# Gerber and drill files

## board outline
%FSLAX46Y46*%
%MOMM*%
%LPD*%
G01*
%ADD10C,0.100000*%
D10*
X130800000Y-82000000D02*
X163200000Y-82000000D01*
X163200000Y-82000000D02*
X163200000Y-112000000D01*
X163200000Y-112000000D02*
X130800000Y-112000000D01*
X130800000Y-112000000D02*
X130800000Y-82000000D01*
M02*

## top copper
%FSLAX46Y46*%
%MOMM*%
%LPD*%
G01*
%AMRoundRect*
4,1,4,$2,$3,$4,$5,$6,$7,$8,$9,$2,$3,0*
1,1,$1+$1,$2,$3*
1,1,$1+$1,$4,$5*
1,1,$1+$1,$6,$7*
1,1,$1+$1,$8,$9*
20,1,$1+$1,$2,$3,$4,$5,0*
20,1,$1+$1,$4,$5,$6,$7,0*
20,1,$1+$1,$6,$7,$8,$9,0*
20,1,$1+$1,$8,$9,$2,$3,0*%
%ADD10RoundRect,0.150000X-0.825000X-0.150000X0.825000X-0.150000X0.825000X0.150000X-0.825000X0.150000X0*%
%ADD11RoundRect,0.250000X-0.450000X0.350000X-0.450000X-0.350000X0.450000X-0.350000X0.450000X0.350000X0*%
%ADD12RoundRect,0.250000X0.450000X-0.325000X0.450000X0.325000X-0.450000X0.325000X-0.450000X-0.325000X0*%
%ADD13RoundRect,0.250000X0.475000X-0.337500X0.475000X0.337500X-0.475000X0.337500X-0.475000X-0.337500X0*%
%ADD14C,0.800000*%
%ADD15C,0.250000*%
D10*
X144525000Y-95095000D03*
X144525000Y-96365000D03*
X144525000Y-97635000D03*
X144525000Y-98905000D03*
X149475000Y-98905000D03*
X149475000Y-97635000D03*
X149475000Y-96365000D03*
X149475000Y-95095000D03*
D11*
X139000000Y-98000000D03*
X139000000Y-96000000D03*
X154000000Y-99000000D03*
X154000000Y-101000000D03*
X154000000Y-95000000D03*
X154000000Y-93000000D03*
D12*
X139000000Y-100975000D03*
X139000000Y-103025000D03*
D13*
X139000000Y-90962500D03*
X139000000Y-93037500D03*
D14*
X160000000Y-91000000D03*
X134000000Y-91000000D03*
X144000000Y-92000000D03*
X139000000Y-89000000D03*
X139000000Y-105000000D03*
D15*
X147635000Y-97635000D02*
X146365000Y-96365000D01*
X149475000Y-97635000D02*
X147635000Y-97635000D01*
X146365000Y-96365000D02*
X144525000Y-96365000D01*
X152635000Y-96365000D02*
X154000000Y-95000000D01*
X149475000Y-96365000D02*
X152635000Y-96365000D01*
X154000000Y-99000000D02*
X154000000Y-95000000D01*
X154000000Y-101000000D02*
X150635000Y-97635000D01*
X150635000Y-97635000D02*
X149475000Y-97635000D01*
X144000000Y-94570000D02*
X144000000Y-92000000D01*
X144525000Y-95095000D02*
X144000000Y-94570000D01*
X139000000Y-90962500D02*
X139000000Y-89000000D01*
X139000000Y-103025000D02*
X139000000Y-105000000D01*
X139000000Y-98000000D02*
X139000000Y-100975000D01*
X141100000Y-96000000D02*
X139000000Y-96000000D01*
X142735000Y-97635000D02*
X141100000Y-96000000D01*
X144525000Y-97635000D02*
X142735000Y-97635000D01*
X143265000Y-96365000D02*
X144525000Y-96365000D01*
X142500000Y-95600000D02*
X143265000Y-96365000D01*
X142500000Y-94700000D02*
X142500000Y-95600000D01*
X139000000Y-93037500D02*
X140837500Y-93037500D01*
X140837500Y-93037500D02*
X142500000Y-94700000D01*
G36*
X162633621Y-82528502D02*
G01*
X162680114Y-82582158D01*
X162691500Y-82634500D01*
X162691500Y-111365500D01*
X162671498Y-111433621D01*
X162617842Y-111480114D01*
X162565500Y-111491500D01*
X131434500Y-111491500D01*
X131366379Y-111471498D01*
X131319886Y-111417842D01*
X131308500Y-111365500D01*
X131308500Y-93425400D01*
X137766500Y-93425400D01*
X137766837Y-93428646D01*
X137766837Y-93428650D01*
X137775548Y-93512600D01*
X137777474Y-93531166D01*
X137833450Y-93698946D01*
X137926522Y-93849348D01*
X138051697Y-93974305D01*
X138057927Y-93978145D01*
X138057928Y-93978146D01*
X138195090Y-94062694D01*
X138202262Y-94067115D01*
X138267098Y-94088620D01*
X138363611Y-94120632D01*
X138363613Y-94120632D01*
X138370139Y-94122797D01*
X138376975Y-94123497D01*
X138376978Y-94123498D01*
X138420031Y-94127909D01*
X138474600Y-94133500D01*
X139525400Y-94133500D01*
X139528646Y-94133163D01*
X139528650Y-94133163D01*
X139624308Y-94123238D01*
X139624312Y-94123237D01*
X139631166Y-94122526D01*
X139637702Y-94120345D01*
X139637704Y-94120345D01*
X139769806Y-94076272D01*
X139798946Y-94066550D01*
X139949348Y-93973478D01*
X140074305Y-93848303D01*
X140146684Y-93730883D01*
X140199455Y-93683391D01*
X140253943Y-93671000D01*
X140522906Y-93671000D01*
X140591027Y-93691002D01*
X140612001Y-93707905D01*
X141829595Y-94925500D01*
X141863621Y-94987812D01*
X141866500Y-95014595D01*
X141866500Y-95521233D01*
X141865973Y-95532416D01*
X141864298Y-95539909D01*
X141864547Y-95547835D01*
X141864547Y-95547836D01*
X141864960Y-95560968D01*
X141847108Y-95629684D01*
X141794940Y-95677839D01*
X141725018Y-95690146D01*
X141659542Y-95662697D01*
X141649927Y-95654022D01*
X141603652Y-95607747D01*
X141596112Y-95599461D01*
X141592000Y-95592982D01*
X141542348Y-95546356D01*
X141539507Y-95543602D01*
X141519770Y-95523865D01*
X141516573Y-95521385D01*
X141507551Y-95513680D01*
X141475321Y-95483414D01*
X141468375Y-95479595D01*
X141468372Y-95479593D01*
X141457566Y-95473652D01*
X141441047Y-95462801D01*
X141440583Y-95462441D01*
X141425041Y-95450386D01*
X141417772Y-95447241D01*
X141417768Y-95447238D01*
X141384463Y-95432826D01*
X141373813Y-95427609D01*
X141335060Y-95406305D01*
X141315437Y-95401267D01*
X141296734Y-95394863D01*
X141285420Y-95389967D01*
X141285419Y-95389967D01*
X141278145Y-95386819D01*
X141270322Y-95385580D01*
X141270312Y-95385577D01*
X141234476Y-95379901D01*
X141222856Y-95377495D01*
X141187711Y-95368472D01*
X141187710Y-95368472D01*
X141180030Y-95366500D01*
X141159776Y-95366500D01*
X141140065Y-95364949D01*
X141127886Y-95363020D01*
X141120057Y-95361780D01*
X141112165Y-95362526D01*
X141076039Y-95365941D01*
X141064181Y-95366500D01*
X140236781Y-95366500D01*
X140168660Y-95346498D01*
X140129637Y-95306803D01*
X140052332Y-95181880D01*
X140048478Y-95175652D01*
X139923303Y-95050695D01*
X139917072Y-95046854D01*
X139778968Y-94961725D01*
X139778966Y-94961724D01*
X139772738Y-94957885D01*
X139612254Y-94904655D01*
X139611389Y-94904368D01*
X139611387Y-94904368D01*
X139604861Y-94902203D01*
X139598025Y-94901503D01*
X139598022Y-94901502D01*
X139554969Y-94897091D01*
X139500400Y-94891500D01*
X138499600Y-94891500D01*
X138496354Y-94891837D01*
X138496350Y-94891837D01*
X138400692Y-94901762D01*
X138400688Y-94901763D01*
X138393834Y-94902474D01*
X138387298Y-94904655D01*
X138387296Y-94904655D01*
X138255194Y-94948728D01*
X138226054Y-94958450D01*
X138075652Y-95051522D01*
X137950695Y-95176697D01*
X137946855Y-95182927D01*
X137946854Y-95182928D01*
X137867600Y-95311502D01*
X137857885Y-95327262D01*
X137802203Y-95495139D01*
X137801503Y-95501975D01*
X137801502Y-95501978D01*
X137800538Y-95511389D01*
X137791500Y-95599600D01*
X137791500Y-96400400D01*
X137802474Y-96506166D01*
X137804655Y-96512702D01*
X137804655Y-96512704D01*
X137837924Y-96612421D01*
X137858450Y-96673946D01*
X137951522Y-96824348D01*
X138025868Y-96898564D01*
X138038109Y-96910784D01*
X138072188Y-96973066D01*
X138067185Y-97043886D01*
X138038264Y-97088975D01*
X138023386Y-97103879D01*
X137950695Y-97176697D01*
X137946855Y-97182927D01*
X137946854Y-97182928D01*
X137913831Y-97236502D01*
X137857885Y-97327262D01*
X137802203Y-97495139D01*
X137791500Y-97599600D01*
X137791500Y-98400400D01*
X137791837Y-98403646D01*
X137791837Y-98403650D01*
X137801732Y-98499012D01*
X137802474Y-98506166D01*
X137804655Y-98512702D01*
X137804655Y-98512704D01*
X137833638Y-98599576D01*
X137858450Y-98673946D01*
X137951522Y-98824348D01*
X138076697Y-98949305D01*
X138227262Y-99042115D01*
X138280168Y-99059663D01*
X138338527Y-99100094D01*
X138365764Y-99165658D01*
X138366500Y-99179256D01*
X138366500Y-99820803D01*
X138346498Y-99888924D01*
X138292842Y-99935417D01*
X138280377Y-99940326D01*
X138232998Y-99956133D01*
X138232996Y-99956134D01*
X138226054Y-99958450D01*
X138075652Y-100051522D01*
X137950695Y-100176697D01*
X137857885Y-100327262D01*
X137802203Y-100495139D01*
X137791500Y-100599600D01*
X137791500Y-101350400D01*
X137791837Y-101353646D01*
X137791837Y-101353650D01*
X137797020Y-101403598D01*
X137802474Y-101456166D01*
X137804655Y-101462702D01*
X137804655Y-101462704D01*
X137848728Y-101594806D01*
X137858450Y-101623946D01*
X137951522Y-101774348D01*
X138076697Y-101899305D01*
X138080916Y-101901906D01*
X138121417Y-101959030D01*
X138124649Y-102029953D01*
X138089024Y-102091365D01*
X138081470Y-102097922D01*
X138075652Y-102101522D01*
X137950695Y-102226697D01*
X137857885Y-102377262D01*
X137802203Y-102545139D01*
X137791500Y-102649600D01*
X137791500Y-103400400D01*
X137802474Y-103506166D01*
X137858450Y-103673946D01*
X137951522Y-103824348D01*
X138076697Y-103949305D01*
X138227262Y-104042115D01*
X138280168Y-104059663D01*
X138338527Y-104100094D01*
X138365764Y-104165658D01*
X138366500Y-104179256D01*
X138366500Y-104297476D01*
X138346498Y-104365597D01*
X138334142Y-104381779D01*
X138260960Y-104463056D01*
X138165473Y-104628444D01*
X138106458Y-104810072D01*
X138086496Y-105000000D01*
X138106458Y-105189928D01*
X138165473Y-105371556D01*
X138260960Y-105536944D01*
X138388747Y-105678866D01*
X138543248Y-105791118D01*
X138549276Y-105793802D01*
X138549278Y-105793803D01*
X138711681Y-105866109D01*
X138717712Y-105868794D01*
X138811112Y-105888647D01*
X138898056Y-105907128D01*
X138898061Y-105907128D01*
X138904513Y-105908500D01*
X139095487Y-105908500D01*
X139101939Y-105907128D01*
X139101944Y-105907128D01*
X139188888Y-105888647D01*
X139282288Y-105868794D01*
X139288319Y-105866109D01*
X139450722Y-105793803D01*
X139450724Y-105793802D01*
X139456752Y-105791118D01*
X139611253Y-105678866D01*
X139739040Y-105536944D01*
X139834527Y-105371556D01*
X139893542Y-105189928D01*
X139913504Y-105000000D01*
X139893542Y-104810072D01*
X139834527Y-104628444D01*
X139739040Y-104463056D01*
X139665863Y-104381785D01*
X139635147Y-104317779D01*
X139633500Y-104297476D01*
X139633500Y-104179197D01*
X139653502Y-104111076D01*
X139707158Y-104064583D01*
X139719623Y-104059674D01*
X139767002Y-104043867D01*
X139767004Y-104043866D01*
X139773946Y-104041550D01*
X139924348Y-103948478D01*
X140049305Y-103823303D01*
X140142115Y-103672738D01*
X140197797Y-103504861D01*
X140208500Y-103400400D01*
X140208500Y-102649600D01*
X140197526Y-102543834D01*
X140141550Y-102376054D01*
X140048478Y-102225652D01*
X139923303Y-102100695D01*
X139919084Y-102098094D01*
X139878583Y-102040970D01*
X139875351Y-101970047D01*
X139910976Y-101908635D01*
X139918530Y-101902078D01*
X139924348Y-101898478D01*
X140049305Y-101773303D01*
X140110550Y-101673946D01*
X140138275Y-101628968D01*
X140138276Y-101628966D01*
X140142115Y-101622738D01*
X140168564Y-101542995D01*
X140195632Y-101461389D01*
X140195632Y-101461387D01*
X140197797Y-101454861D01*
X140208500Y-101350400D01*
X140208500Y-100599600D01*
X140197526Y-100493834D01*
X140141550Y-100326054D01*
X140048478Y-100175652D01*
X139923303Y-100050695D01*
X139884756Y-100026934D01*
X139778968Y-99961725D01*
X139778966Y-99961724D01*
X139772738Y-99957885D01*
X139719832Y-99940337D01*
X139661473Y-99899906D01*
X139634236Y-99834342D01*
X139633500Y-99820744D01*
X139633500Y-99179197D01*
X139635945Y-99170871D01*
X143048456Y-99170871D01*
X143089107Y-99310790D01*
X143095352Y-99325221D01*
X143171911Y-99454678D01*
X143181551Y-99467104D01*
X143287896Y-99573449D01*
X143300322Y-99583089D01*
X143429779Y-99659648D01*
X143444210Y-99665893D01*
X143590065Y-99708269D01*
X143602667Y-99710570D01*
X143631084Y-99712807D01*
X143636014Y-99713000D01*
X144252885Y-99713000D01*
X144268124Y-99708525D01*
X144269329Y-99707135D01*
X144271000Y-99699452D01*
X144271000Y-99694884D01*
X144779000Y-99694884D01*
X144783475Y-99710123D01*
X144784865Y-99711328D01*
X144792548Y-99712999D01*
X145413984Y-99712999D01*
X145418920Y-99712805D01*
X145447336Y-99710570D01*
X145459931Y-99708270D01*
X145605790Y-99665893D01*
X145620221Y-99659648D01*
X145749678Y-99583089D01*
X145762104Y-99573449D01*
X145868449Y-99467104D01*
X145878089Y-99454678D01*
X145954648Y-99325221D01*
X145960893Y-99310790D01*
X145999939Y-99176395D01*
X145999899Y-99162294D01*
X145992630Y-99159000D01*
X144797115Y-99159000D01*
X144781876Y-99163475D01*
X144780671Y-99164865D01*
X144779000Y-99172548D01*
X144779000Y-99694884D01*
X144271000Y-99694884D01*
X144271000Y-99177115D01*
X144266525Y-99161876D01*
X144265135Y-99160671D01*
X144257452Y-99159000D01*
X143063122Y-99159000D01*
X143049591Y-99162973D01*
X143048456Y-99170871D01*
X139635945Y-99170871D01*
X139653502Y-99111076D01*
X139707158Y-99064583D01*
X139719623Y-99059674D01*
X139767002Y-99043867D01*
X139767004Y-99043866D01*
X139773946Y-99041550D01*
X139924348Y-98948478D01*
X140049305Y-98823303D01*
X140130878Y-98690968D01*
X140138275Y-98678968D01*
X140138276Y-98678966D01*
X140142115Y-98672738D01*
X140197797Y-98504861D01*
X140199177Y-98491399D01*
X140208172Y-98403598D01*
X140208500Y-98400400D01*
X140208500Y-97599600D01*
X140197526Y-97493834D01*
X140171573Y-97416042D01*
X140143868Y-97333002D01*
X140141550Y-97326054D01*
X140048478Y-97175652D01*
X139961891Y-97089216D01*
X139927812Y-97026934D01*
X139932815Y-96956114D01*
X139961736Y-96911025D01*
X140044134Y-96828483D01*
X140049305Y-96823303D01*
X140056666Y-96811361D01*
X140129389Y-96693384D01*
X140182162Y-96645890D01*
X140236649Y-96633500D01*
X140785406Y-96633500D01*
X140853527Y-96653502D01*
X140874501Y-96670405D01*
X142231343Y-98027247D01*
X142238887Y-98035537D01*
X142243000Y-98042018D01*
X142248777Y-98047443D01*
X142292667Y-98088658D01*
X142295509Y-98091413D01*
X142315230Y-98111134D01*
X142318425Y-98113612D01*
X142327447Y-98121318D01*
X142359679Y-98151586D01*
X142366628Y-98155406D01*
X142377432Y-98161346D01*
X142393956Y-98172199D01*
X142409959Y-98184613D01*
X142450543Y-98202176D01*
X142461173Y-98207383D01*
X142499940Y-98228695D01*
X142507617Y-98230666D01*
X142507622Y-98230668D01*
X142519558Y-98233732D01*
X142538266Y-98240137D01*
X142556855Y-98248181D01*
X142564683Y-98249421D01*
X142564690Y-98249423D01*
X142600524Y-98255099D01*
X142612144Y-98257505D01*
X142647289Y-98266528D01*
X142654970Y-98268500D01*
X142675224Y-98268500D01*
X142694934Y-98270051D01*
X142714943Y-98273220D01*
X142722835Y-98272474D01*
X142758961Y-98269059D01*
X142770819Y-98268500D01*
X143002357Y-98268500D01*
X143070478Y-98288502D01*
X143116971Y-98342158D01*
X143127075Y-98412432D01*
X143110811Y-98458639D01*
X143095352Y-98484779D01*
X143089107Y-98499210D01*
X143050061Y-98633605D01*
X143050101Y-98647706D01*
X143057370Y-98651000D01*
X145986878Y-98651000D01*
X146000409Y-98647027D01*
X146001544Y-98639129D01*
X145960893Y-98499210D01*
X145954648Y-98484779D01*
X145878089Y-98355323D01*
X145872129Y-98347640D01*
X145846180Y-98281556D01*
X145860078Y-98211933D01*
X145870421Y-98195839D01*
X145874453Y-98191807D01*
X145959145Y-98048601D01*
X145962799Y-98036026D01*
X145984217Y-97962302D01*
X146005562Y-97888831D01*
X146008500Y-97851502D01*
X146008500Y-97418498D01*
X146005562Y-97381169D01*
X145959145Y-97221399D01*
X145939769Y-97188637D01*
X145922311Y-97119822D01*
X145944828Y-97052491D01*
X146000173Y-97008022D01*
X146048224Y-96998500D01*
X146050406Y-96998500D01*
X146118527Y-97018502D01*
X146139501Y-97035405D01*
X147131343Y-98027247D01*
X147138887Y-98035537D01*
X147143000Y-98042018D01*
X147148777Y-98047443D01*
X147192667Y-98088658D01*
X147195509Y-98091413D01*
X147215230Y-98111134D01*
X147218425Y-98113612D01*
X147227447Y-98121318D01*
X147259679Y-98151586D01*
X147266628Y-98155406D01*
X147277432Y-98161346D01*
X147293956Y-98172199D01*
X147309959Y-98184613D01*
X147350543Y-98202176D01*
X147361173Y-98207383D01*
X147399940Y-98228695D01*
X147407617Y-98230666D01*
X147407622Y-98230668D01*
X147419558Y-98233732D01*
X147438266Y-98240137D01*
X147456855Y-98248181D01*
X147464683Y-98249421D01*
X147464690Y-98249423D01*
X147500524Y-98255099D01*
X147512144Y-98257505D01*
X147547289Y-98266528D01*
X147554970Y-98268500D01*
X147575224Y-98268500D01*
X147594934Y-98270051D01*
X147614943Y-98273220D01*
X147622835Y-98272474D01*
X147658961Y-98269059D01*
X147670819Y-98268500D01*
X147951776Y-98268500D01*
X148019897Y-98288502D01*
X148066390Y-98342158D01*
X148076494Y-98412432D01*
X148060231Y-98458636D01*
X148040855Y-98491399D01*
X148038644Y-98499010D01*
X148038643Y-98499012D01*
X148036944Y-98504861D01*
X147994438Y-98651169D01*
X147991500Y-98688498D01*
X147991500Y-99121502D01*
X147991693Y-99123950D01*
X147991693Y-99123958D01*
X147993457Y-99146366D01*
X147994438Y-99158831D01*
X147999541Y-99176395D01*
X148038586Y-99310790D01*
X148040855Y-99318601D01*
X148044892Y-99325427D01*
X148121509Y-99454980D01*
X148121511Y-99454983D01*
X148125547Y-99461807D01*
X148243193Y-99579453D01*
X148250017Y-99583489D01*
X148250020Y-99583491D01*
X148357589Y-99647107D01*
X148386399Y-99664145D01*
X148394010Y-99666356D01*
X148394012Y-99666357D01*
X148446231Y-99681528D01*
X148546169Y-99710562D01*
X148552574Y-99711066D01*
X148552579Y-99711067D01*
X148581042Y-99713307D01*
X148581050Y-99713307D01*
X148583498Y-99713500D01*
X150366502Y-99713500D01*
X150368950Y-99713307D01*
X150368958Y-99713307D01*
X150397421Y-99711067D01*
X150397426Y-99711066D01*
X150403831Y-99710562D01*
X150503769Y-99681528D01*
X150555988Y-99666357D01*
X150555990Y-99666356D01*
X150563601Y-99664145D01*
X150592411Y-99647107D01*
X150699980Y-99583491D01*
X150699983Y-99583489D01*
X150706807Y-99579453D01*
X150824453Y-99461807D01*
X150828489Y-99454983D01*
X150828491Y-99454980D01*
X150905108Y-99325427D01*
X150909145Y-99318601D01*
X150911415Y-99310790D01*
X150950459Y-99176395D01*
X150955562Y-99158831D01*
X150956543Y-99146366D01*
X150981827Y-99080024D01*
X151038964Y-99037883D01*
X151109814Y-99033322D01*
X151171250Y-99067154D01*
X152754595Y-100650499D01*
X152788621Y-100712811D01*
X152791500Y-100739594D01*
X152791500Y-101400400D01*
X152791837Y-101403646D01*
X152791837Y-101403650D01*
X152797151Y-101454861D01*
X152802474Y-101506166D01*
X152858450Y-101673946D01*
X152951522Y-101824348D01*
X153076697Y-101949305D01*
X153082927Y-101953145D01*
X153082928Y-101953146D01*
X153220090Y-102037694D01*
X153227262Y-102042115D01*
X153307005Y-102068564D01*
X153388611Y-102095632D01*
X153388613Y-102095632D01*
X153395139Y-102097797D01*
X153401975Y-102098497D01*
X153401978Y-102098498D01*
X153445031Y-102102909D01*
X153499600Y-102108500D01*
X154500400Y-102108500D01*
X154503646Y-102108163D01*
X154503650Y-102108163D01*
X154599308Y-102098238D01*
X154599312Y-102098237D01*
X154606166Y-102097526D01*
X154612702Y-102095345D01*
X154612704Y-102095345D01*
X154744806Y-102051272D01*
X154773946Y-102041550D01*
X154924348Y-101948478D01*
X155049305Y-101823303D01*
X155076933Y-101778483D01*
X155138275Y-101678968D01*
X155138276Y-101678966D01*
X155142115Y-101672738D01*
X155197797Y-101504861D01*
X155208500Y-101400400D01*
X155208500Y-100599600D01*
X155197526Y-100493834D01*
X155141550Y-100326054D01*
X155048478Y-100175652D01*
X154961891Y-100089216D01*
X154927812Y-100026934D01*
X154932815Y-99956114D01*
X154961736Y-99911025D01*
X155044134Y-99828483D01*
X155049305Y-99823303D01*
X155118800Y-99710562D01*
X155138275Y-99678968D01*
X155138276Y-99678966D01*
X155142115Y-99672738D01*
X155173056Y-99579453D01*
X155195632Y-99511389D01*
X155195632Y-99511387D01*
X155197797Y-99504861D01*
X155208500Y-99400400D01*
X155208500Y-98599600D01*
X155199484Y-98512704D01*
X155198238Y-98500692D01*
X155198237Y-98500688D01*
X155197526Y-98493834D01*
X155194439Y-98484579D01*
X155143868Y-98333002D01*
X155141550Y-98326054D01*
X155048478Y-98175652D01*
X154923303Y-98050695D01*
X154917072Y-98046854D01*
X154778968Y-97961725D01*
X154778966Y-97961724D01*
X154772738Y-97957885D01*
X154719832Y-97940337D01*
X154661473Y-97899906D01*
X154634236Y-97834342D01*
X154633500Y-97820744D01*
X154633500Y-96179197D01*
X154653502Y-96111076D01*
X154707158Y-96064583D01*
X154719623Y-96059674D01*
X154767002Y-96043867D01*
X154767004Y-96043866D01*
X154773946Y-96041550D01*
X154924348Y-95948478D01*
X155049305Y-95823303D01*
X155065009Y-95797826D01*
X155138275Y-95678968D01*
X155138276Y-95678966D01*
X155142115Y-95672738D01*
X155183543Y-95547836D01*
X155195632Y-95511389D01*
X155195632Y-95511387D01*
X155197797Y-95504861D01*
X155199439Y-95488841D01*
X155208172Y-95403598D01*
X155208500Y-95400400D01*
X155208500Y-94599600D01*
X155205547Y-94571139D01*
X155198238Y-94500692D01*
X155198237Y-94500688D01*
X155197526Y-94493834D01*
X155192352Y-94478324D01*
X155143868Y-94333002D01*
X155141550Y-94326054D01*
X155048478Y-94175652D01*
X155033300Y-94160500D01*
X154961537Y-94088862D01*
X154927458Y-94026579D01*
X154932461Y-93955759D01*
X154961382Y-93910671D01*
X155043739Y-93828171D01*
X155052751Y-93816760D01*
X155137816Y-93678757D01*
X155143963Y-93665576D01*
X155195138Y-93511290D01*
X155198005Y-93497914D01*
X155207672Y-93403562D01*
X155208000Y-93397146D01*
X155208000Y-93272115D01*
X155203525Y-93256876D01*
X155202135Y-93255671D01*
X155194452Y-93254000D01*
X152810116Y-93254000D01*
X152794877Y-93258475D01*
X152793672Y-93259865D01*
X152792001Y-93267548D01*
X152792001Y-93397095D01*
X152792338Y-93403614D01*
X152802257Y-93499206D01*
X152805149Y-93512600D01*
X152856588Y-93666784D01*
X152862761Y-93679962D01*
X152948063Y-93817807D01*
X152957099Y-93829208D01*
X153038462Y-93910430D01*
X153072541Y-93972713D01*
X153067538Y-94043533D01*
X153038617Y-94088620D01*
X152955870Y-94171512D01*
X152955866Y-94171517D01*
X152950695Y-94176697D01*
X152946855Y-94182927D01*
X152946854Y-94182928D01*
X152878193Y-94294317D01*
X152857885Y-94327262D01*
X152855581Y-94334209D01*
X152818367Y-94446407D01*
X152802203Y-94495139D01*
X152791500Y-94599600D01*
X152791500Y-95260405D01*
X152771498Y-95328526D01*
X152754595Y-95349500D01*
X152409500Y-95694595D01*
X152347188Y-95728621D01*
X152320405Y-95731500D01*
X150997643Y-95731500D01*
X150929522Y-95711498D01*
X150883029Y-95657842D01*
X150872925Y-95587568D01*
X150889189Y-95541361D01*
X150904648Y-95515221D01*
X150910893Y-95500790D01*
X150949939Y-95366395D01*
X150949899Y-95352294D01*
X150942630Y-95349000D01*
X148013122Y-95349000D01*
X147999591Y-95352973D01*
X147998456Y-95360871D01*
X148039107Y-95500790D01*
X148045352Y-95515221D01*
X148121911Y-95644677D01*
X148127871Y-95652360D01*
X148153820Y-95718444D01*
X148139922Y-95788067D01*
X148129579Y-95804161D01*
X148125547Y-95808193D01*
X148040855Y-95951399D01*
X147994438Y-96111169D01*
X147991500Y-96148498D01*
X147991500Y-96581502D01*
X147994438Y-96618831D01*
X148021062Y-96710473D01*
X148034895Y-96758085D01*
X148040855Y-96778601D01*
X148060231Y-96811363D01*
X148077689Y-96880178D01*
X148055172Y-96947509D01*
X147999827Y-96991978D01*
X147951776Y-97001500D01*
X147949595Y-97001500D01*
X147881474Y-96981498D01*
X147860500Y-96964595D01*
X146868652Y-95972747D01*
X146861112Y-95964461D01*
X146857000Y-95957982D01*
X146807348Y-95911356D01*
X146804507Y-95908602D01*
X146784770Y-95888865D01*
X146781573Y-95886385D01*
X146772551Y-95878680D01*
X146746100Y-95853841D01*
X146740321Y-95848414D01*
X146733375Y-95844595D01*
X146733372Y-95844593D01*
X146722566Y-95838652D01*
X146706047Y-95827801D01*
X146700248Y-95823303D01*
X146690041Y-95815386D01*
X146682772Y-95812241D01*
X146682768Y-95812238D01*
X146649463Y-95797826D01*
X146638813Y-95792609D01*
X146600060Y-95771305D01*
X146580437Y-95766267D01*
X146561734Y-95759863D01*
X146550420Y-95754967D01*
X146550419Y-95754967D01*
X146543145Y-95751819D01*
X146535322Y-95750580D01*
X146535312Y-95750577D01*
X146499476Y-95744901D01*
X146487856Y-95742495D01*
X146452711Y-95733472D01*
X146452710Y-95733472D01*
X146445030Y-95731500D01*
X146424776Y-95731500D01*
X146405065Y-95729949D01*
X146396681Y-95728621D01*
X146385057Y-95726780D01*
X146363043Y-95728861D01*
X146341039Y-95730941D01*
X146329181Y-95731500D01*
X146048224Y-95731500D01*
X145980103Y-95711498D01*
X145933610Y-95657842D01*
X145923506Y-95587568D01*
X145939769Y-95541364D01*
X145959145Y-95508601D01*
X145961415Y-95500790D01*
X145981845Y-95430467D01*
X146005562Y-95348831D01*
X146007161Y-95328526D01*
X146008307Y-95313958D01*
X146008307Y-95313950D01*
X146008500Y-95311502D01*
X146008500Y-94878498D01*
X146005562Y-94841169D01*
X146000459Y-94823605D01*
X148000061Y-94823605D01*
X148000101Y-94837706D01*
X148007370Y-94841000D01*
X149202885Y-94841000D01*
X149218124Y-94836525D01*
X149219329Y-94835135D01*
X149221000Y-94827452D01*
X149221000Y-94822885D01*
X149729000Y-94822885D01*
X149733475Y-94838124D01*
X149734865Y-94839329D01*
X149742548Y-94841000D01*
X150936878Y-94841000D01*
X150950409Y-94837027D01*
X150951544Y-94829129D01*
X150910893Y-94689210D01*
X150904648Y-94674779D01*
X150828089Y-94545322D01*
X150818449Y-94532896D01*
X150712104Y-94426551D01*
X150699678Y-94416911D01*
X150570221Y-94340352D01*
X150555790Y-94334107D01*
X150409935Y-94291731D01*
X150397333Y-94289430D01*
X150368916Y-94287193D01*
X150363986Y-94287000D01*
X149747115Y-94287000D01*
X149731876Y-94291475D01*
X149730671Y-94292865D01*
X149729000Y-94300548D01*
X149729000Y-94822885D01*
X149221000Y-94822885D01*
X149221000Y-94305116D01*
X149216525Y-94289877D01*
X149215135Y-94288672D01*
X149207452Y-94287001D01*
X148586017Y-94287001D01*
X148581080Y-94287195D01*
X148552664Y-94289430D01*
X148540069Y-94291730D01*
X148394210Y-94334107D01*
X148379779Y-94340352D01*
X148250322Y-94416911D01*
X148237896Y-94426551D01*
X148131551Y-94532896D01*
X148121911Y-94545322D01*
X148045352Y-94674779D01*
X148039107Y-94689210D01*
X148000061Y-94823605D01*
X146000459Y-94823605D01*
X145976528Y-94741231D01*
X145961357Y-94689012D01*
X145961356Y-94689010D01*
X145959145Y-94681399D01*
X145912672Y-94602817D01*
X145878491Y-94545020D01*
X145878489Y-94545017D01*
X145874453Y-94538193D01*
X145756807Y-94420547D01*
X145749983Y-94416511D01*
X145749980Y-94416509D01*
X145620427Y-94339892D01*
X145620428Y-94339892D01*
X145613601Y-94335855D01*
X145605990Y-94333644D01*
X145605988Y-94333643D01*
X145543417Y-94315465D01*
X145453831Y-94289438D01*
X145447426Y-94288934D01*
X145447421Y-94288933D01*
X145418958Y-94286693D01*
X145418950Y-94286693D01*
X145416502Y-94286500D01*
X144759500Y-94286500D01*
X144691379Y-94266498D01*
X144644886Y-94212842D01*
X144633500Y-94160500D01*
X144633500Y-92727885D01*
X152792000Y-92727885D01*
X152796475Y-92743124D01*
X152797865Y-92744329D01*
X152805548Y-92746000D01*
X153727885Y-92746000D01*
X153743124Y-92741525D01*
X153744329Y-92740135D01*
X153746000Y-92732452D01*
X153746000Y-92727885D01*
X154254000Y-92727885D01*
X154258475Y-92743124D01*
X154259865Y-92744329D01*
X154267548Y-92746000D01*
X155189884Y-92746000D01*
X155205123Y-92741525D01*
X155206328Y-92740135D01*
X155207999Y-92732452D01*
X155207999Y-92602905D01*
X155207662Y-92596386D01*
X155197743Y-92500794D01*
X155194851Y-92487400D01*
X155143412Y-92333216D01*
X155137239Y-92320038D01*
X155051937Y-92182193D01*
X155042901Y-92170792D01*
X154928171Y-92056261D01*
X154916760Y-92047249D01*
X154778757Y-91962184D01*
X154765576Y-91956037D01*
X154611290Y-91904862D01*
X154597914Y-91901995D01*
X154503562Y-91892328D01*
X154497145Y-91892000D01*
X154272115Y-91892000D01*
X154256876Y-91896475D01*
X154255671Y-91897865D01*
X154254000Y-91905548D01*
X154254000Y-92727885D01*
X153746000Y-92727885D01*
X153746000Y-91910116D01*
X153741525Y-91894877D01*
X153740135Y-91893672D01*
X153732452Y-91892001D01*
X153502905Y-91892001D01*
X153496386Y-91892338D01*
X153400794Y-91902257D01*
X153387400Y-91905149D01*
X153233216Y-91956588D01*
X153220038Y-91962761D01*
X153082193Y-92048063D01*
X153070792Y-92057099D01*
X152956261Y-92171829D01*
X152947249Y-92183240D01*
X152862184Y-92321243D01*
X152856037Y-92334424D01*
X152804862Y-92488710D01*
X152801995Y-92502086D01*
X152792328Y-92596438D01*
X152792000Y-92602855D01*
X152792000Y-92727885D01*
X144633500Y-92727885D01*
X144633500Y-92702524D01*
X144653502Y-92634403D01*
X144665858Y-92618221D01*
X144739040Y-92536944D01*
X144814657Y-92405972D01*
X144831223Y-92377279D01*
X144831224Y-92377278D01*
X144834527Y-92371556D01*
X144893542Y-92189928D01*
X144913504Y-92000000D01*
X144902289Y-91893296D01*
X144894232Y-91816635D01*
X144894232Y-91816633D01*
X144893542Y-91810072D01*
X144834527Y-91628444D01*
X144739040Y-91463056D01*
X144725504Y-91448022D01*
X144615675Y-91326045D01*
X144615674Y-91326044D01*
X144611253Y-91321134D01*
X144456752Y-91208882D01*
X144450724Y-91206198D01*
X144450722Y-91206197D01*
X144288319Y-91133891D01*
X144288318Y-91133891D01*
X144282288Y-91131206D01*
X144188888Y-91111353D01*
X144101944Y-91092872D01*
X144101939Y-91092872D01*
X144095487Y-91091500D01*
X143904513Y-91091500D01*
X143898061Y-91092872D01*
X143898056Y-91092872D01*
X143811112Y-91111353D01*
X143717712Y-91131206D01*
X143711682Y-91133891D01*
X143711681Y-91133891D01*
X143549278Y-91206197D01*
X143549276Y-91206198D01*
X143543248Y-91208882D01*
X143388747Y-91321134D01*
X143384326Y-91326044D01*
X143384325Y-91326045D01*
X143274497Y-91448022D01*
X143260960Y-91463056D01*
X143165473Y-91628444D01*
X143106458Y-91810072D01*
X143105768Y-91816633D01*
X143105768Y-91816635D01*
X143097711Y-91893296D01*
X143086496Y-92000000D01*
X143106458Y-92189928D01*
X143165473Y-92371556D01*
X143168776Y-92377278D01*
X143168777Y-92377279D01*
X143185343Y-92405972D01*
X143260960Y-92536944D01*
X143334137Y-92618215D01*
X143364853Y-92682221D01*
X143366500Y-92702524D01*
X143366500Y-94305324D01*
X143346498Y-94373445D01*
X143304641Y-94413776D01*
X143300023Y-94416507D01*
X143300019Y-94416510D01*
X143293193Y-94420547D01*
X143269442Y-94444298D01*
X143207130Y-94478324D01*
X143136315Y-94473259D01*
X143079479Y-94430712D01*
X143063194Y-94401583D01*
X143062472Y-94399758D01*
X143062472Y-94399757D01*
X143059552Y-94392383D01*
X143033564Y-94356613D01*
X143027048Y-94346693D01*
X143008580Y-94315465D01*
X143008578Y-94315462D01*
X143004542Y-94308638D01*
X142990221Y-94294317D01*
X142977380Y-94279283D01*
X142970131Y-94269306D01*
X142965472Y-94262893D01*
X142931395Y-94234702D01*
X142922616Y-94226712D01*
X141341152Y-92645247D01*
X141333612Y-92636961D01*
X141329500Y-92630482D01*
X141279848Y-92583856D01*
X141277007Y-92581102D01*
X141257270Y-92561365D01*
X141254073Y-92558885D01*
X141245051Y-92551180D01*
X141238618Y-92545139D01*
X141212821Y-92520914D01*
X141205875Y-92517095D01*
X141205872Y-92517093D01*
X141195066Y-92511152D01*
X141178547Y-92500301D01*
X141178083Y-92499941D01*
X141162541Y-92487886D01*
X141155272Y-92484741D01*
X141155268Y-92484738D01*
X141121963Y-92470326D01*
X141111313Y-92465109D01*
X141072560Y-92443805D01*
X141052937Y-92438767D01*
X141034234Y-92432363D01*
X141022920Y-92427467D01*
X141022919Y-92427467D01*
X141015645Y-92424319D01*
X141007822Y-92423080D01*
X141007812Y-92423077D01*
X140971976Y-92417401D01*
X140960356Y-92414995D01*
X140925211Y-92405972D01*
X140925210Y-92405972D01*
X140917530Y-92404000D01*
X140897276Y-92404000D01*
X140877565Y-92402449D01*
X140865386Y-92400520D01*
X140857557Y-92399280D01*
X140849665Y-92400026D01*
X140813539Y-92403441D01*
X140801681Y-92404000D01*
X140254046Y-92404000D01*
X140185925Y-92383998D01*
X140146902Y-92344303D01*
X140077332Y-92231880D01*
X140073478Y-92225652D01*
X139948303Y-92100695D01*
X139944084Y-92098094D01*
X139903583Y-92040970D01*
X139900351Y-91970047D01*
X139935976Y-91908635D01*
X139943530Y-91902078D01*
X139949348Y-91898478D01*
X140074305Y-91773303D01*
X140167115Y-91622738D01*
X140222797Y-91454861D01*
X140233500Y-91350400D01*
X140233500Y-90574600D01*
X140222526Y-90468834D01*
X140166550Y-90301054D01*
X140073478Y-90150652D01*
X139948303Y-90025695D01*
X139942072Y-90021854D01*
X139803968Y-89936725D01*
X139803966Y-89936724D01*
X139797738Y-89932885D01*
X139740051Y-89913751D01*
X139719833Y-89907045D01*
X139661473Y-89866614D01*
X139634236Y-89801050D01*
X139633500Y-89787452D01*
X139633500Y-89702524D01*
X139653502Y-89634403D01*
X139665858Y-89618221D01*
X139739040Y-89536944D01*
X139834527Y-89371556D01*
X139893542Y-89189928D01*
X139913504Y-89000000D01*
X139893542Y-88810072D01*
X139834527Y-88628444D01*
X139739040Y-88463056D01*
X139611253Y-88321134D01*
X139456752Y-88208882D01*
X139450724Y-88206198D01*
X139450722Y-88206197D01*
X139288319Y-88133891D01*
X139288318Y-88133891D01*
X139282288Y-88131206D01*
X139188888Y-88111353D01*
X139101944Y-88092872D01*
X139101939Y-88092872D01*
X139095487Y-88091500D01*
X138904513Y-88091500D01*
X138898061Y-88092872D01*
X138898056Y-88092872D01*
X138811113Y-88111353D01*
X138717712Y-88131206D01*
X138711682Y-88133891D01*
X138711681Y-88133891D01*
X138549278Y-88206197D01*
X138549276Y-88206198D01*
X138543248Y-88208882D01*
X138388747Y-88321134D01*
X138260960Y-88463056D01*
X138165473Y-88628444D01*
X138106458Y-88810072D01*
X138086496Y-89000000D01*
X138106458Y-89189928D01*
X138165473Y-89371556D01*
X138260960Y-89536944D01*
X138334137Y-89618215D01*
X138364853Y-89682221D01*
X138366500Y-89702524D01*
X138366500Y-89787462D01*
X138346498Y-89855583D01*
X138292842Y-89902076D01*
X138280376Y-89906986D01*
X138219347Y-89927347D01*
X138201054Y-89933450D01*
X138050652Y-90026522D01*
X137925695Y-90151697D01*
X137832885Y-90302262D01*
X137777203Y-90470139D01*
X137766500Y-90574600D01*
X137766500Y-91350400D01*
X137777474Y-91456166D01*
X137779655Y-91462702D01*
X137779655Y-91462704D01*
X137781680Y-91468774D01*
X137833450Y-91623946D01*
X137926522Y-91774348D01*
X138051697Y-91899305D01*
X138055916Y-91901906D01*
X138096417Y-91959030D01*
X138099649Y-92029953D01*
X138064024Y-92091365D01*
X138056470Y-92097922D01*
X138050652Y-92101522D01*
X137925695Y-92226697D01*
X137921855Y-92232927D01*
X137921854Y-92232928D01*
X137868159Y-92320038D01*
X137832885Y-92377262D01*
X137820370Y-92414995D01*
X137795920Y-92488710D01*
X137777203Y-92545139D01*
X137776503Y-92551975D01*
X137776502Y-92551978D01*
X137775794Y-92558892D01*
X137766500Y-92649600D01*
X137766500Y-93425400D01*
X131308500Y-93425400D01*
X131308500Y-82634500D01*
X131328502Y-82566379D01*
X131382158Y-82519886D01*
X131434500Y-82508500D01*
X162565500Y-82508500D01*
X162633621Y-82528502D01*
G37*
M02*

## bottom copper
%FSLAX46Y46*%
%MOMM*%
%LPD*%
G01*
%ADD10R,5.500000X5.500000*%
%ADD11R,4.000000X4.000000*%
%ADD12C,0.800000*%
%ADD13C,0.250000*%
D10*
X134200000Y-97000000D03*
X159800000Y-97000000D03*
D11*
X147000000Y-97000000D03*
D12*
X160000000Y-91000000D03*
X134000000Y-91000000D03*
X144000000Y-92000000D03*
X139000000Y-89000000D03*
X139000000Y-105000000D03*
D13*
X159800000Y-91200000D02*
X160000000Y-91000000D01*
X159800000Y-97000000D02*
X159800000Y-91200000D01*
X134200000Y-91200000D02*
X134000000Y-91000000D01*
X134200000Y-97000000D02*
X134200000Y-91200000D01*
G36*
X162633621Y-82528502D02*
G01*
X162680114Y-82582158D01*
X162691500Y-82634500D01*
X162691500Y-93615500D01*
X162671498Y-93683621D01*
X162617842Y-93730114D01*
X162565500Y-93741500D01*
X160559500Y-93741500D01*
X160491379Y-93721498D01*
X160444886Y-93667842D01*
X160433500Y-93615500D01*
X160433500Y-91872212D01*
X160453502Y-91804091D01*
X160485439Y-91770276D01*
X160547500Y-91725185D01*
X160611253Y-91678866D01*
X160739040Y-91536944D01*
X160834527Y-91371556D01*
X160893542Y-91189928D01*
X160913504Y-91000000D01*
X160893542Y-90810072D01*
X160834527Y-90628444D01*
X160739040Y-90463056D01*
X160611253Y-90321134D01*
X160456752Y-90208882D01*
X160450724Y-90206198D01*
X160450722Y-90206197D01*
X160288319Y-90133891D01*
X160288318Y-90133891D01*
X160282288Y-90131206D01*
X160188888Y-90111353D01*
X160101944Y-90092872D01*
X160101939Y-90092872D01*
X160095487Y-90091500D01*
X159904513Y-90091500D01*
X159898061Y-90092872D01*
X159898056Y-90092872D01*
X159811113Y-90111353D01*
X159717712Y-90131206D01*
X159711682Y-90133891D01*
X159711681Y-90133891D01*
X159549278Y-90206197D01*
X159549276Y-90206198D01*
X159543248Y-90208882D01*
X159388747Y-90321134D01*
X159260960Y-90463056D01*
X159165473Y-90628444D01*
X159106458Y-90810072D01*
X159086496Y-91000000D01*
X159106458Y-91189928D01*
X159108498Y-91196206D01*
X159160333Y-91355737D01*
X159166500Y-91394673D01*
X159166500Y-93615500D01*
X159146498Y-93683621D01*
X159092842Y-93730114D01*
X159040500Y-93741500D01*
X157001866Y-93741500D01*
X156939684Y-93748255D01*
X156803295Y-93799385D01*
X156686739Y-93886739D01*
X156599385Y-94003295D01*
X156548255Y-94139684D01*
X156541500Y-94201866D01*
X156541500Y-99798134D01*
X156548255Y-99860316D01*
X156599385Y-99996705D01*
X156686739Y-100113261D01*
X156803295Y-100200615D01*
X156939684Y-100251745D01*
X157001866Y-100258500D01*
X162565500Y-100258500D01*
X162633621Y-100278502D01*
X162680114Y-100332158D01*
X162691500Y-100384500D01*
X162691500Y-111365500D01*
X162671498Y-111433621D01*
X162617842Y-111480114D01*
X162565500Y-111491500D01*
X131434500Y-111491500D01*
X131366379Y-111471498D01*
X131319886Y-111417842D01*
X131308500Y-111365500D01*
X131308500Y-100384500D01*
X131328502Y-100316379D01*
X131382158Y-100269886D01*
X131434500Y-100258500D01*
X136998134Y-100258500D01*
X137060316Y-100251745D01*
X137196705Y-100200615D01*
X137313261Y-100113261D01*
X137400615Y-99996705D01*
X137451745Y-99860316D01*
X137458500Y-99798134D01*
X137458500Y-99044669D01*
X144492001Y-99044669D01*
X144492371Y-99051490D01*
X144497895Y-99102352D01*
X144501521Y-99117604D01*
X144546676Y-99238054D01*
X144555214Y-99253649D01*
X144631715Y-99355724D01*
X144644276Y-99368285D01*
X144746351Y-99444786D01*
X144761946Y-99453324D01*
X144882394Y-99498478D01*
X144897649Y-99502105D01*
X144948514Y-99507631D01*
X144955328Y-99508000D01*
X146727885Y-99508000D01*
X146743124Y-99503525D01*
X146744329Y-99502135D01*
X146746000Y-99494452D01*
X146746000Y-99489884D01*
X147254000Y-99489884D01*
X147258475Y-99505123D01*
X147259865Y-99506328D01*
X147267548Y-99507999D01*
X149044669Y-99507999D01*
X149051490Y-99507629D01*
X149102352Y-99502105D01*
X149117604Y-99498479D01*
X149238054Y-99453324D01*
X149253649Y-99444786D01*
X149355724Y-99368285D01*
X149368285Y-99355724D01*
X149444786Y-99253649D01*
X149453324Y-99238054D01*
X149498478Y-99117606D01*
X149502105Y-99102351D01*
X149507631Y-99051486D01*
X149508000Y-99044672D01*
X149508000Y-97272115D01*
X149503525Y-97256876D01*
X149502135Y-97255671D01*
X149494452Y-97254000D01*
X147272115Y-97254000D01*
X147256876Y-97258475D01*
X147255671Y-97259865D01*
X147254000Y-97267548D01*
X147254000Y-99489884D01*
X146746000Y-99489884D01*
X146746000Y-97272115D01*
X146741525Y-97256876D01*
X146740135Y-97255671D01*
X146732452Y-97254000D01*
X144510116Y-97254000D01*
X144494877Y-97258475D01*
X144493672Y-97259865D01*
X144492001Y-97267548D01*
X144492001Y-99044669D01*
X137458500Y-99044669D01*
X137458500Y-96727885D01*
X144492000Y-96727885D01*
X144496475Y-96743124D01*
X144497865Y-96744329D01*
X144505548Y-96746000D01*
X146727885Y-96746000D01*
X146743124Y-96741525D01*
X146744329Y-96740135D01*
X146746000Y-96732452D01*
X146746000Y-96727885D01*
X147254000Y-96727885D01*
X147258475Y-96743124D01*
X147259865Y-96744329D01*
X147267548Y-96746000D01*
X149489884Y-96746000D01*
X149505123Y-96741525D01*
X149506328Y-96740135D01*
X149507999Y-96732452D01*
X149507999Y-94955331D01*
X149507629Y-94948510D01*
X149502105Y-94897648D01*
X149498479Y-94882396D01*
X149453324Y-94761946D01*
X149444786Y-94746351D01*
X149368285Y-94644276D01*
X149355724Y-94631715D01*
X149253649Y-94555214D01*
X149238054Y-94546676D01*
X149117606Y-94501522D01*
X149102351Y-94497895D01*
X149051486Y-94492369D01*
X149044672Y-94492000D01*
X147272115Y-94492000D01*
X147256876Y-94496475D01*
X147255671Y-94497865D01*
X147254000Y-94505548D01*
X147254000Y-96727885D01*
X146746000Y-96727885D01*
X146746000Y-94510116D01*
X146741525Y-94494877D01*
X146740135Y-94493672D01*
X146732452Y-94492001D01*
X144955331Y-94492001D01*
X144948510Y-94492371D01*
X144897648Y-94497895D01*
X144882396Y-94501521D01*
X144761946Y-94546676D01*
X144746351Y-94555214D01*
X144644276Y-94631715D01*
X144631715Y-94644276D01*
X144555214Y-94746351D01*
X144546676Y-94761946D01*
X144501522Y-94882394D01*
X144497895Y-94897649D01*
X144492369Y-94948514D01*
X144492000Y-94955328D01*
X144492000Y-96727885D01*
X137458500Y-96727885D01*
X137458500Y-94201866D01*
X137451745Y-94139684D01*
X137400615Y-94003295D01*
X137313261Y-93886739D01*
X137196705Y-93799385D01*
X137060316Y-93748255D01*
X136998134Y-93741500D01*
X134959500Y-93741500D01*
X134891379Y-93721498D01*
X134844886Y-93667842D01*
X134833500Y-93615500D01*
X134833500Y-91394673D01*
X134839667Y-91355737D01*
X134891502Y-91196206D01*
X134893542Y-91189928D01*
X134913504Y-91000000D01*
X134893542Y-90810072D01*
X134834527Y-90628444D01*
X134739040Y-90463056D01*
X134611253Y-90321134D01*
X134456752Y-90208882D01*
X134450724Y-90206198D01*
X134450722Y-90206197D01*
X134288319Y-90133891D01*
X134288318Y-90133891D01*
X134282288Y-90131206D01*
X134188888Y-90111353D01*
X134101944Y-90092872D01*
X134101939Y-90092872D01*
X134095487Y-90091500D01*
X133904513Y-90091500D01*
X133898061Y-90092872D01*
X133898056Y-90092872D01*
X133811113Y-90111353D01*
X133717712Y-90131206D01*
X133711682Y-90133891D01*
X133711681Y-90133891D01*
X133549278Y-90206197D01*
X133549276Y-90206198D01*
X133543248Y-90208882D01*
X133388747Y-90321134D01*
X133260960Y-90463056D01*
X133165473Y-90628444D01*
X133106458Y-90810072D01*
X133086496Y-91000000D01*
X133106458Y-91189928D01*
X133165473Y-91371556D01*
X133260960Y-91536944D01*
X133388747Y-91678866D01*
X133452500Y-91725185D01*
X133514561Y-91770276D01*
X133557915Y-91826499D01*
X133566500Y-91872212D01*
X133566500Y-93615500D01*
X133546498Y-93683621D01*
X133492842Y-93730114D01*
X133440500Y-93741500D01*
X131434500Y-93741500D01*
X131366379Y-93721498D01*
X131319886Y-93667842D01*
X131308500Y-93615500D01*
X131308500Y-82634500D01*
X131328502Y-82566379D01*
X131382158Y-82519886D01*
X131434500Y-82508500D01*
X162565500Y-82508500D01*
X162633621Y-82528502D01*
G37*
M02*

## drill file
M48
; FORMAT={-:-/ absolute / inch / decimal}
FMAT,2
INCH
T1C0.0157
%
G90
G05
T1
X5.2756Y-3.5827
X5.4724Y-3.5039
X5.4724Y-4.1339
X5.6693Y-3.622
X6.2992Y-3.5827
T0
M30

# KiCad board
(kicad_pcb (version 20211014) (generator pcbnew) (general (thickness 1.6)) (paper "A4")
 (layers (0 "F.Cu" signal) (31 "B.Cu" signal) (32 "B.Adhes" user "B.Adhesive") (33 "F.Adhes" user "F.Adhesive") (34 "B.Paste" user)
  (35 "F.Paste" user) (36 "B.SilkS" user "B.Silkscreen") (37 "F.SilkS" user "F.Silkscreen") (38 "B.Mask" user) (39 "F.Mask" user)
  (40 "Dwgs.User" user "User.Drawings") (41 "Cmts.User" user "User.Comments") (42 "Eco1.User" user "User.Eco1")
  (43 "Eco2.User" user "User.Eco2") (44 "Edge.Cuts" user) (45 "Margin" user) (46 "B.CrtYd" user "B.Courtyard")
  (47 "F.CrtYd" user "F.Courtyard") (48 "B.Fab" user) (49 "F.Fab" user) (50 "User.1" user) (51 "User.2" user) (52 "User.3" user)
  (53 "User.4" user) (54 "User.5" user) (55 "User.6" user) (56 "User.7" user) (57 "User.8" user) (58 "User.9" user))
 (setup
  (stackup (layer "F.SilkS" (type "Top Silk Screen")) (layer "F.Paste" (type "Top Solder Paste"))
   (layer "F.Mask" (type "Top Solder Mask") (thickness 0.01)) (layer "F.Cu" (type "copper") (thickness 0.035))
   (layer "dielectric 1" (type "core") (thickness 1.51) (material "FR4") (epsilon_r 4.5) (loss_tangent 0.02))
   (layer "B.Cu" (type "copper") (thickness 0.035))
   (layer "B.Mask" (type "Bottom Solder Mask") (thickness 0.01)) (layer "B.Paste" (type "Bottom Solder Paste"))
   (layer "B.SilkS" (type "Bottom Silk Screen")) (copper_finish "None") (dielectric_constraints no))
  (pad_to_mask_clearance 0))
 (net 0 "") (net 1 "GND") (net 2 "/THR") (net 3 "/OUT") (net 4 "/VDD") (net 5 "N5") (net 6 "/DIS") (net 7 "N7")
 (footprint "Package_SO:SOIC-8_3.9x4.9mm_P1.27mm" (layer "F.Cu") (at 147 97)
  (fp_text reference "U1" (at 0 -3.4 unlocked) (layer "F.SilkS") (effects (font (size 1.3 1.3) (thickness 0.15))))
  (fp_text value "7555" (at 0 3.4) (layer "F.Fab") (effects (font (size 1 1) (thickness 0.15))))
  (pad "1" smd roundrect (at -2.475 -1.905) (size 1.95 0.6) (layers "F.Cu" "F.Paste" "F.Mask") (roundrect_rratio 0.25) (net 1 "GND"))
  (pad "2" smd roundrect (at -2.475 -0.635) (size 1.95 0.6) (layers "F.Cu" "F.Paste" "F.Mask") (roundrect_rratio 0.25) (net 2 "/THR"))
  (pad "3" smd roundrect (at -2.475 0.635) (size 1.95 0.6) (layers "F.Cu" "F.Paste" "F.Mask") (roundrect_rratio 0.25) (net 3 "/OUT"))
  (pad "4" smd roundrect (at -2.475 1.905) (size 1.95 0.6) (layers "F.Cu" "F.Paste" "F.Mask") (roundrect_rratio 0.25) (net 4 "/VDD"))
  (pad "5" smd roundrect (at 2.475 1.905) (size 1.95 0.6) (layers "F.Cu" "F.Paste" "F.Mask") (roundrect_rratio 0.25) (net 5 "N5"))
  (pad "6" smd roundrect (at 2.475 0.635) (size 1.95 0.6) (layers "F.Cu" "F.Paste" "F.Mask") (roundrect_rratio 0.25) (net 2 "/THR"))
  (pad "7" smd roundrect (at 2.475 -0.635) (size 1.95 0.6) (layers "F.Cu" "F.Paste" "F.Mask") (roundrect_rratio 0.25) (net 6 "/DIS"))
  (pad "8" smd roundrect (at 2.475 -1.905) (size 1.95 0.6) (layers "F.Cu" "F.Paste" "F.Mask") (roundrect_rratio 0.25) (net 4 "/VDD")))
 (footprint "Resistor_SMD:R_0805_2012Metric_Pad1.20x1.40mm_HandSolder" (layer "F.Cu") (at 154 94 -90)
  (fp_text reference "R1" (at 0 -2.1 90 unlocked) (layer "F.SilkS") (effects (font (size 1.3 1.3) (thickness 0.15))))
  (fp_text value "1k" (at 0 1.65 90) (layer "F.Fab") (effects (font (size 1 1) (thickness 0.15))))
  (pad "1" smd roundrect (at -1 0 270) (size 1.2 1.4) (layers "F.Cu" "F.Paste" "F.Mask") (roundrect_rratio 0.2083333333) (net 4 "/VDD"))
  (pad "2" smd roundrect (at 1 0 270) (size 1.2 1.4) (layers "F.Cu" "F.Paste" "F.Mask") (roundrect_rratio 0.2083333333) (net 6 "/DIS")))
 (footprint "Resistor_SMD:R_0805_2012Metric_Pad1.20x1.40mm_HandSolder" (layer "F.Cu") (at 139 97 -90)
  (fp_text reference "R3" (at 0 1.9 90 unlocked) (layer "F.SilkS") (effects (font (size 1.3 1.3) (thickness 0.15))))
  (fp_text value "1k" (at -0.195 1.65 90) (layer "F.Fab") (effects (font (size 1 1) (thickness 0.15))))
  (pad "1" smd roundrect (at -1 0 270) (size 1.2 1.4) (layers "F.Cu" "F.Paste" "F.Mask") (roundrect_rratio 0.2083333333) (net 3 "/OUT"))
  (pad "2" smd roundrect (at 1 0 270) (size 1.2 1.4) (layers "F.Cu" "F.Paste" "F.Mask") (roundrect_rratio 0.2083333333) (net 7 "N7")))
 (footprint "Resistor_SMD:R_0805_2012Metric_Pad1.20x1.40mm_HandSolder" (layer "F.Cu") (at 154 100 -90)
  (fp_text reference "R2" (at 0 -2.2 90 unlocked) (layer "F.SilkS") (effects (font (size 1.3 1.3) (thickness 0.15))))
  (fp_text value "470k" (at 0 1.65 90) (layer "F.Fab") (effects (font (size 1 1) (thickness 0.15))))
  (pad "1" smd roundrect (at -1 0 270) (size 1.2 1.4) (layers "F.Cu" "F.Paste" "F.Mask") (roundrect_rratio 0.2083333333) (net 6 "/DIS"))
  (pad "2" smd roundrect (at 1 0 270) (size 1.2 1.4) (layers "F.Cu" "F.Paste" "F.Mask") (roundrect_rratio 0.2083333333) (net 2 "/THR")))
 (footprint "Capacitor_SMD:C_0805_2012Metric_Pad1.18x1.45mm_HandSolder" (layer "F.Cu") (at 139 92 90)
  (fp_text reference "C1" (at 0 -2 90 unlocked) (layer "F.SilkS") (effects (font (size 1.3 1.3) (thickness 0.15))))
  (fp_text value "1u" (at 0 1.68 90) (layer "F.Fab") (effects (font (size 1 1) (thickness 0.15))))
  (pad "1" smd roundrect (at -1.0375 0 90) (size 1.175 1.45) (layers "F.Cu" "F.Paste" "F.Mask") (roundrect_rratio 0.2127659574)
   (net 2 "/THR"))
  (pad "2" smd roundrect (at 1.0375 0 90) (size 1.175 1.45) (layers "F.Cu" "F.Paste" "F.Mask") (roundrect_rratio 0.2127659574) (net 1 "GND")))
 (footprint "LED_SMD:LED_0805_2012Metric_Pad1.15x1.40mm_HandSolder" (layer "F.Cu") (at 139 102 90)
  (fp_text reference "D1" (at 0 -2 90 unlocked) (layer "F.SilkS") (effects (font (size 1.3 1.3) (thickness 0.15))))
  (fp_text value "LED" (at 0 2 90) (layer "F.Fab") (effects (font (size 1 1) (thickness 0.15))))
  (pad "1" smd roundrect (at -1.025 0 90) (size 1.15 1.4) (layers "F.Cu" "F.Paste" "F.Mask") (roundrect_rratio 0.2173913043) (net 1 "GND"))
  (pad "2" smd roundrect (at 1.025 0 90) (size 1.15 1.4) (layers "F.Cu" "F.Paste" "F.Mask") (roundrect_rratio 0.2173913043) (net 7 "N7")))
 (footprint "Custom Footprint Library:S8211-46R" (layer "B.Cu") (at 147 97 180)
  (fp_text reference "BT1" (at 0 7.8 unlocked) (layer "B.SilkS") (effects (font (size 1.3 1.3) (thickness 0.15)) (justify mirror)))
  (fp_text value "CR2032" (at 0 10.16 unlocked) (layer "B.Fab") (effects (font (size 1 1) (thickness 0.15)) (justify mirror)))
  (pad "1" smd rect (at -12.8 0 180) (size 5.5 5.5) (layers "B.Cu" "B.Paste" "B.Mask") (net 4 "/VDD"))
  (pad "1" smd rect (at 12.8 0 180) (size 5.5 5.5) (layers "B.Cu" "B.Paste" "B.Mask") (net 4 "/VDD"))
  (pad "2" smd rect (at 0 0 180) (size 4 4) (layers "B.Cu" "B.Paste" "B.Mask") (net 1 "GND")))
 (gr_rect (start 130.8 82) (end 163.2 112) (layer "Edge.Cuts") (width 0.1) (fill none))
 (segment (start 144.525 95.095) (end 144 94.57) (width 0.25) (layer "F.Cu") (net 1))
 (segment (start 144 94.57) (end 144 92) (width 0.25) (layer "F.Cu") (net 1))
 (segment (start 139 90.9625) (end 139 89) (width 0.25) (layer "F.Cu") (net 1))
 (segment (start 139 103.025) (end 139 105) (width 0.25) (layer "F.Cu") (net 1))
 (via (at 139 89) (size 0.8) (drill 0.4) (layers "F.Cu" "B.Cu") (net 1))
 (via (at 139 105) (size 0.8) (drill 0.4) (layers "F.Cu" "B.Cu") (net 1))
 (via (at 144 92) (size 0.8) (drill 0.4) (layers "F.Cu" "B.Cu") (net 1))
 (segment (start 139 98) (end 139 100.975) (width 0.25) (layer "F.Cu") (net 7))
 (via (at 134 91) (size 0.8) (drill 0.4) (layers "F.Cu" "B.Cu") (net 4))
 (via (at 160 91) (size 0.8) (drill 0.4) (layers "F.Cu" "B.Cu") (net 4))
 (segment (start 159.8 91.2) (end 160 91) (width 0.25) (layer "B.Cu") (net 4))
 (segment (start 134.2 97) (end 134.2 91.2) (width 0.25) (layer "B.Cu") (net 4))
 (segment (start 159.8 97) (end 159.8 91.2) (width 0.25) (layer "B.Cu") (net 4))
 (segment (start 134.2 91.2) (end 134 91) (width 0.25) (layer "B.Cu") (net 4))
 (segment (start 142.5 95.6) (end 143.265 96.365) (width 0.25) (layer "F.Cu") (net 2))
 (segment (start 149.475 97.635) (end 147.635 97.635) (width 0.25) (layer "F.Cu") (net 2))
 (segment (start 143.265 96.365) (end 144.525 96.365) (width 0.25) (layer "F.Cu") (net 2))
 (segment (start 139 93.0375) (end 140.8375 93.0375) (width 0.25) (layer "F.Cu") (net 2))
 (segment (start 150.635 97.635) (end 149.475 97.635) (width 0.25) (layer "F.Cu") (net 2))
 (segment (start 142.5 94.7) (end 142.5 95.6) (width 0.25) (layer "F.Cu") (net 2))
 (segment (start 146.365 96.365) (end 144.525 96.365) (width 0.25) (layer "F.Cu") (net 2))
 (segment (start 140.8375 93.0375) (end 142.5 94.7) (width 0.25) (layer "F.Cu") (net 2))
 (segment (start 147.635 97.635) (end 146.365 96.365) (width 0.25) (layer "F.Cu") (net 2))
 (segment (start 154 101) (end 150.635 97.635) (width 0.25) (layer "F.Cu") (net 2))
 (segment (start 152.635 96.365) (end 154 95) (width 0.25) (layer "F.Cu") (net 6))
 (segment (start 149.475 96.365) (end 152.635 96.365) (width 0.25) (layer "F.Cu") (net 6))
 (segment (start 154 99) (end 154 95) (width 0.25) (layer "F.Cu") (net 6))
 (segment (start 141.1 96) (end 139 96) (width 0.25) (layer "F.Cu") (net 3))
 (segment (start 144.525 97.635) (end 142.735 97.635) (width 0.25) (layer "F.Cu") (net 3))
 (segment (start 142.735 97.635) (end 141.1 96) (width 0.25) (layer "F.Cu") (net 3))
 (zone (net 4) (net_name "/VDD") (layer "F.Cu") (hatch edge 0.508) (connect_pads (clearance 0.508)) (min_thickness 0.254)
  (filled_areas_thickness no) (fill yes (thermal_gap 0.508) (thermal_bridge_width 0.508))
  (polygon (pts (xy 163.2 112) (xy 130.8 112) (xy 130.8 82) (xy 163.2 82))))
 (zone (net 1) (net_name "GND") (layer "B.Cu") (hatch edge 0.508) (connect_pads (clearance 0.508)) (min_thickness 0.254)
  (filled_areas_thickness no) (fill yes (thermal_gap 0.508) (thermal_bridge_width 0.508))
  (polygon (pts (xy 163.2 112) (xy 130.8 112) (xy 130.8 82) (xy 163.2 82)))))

